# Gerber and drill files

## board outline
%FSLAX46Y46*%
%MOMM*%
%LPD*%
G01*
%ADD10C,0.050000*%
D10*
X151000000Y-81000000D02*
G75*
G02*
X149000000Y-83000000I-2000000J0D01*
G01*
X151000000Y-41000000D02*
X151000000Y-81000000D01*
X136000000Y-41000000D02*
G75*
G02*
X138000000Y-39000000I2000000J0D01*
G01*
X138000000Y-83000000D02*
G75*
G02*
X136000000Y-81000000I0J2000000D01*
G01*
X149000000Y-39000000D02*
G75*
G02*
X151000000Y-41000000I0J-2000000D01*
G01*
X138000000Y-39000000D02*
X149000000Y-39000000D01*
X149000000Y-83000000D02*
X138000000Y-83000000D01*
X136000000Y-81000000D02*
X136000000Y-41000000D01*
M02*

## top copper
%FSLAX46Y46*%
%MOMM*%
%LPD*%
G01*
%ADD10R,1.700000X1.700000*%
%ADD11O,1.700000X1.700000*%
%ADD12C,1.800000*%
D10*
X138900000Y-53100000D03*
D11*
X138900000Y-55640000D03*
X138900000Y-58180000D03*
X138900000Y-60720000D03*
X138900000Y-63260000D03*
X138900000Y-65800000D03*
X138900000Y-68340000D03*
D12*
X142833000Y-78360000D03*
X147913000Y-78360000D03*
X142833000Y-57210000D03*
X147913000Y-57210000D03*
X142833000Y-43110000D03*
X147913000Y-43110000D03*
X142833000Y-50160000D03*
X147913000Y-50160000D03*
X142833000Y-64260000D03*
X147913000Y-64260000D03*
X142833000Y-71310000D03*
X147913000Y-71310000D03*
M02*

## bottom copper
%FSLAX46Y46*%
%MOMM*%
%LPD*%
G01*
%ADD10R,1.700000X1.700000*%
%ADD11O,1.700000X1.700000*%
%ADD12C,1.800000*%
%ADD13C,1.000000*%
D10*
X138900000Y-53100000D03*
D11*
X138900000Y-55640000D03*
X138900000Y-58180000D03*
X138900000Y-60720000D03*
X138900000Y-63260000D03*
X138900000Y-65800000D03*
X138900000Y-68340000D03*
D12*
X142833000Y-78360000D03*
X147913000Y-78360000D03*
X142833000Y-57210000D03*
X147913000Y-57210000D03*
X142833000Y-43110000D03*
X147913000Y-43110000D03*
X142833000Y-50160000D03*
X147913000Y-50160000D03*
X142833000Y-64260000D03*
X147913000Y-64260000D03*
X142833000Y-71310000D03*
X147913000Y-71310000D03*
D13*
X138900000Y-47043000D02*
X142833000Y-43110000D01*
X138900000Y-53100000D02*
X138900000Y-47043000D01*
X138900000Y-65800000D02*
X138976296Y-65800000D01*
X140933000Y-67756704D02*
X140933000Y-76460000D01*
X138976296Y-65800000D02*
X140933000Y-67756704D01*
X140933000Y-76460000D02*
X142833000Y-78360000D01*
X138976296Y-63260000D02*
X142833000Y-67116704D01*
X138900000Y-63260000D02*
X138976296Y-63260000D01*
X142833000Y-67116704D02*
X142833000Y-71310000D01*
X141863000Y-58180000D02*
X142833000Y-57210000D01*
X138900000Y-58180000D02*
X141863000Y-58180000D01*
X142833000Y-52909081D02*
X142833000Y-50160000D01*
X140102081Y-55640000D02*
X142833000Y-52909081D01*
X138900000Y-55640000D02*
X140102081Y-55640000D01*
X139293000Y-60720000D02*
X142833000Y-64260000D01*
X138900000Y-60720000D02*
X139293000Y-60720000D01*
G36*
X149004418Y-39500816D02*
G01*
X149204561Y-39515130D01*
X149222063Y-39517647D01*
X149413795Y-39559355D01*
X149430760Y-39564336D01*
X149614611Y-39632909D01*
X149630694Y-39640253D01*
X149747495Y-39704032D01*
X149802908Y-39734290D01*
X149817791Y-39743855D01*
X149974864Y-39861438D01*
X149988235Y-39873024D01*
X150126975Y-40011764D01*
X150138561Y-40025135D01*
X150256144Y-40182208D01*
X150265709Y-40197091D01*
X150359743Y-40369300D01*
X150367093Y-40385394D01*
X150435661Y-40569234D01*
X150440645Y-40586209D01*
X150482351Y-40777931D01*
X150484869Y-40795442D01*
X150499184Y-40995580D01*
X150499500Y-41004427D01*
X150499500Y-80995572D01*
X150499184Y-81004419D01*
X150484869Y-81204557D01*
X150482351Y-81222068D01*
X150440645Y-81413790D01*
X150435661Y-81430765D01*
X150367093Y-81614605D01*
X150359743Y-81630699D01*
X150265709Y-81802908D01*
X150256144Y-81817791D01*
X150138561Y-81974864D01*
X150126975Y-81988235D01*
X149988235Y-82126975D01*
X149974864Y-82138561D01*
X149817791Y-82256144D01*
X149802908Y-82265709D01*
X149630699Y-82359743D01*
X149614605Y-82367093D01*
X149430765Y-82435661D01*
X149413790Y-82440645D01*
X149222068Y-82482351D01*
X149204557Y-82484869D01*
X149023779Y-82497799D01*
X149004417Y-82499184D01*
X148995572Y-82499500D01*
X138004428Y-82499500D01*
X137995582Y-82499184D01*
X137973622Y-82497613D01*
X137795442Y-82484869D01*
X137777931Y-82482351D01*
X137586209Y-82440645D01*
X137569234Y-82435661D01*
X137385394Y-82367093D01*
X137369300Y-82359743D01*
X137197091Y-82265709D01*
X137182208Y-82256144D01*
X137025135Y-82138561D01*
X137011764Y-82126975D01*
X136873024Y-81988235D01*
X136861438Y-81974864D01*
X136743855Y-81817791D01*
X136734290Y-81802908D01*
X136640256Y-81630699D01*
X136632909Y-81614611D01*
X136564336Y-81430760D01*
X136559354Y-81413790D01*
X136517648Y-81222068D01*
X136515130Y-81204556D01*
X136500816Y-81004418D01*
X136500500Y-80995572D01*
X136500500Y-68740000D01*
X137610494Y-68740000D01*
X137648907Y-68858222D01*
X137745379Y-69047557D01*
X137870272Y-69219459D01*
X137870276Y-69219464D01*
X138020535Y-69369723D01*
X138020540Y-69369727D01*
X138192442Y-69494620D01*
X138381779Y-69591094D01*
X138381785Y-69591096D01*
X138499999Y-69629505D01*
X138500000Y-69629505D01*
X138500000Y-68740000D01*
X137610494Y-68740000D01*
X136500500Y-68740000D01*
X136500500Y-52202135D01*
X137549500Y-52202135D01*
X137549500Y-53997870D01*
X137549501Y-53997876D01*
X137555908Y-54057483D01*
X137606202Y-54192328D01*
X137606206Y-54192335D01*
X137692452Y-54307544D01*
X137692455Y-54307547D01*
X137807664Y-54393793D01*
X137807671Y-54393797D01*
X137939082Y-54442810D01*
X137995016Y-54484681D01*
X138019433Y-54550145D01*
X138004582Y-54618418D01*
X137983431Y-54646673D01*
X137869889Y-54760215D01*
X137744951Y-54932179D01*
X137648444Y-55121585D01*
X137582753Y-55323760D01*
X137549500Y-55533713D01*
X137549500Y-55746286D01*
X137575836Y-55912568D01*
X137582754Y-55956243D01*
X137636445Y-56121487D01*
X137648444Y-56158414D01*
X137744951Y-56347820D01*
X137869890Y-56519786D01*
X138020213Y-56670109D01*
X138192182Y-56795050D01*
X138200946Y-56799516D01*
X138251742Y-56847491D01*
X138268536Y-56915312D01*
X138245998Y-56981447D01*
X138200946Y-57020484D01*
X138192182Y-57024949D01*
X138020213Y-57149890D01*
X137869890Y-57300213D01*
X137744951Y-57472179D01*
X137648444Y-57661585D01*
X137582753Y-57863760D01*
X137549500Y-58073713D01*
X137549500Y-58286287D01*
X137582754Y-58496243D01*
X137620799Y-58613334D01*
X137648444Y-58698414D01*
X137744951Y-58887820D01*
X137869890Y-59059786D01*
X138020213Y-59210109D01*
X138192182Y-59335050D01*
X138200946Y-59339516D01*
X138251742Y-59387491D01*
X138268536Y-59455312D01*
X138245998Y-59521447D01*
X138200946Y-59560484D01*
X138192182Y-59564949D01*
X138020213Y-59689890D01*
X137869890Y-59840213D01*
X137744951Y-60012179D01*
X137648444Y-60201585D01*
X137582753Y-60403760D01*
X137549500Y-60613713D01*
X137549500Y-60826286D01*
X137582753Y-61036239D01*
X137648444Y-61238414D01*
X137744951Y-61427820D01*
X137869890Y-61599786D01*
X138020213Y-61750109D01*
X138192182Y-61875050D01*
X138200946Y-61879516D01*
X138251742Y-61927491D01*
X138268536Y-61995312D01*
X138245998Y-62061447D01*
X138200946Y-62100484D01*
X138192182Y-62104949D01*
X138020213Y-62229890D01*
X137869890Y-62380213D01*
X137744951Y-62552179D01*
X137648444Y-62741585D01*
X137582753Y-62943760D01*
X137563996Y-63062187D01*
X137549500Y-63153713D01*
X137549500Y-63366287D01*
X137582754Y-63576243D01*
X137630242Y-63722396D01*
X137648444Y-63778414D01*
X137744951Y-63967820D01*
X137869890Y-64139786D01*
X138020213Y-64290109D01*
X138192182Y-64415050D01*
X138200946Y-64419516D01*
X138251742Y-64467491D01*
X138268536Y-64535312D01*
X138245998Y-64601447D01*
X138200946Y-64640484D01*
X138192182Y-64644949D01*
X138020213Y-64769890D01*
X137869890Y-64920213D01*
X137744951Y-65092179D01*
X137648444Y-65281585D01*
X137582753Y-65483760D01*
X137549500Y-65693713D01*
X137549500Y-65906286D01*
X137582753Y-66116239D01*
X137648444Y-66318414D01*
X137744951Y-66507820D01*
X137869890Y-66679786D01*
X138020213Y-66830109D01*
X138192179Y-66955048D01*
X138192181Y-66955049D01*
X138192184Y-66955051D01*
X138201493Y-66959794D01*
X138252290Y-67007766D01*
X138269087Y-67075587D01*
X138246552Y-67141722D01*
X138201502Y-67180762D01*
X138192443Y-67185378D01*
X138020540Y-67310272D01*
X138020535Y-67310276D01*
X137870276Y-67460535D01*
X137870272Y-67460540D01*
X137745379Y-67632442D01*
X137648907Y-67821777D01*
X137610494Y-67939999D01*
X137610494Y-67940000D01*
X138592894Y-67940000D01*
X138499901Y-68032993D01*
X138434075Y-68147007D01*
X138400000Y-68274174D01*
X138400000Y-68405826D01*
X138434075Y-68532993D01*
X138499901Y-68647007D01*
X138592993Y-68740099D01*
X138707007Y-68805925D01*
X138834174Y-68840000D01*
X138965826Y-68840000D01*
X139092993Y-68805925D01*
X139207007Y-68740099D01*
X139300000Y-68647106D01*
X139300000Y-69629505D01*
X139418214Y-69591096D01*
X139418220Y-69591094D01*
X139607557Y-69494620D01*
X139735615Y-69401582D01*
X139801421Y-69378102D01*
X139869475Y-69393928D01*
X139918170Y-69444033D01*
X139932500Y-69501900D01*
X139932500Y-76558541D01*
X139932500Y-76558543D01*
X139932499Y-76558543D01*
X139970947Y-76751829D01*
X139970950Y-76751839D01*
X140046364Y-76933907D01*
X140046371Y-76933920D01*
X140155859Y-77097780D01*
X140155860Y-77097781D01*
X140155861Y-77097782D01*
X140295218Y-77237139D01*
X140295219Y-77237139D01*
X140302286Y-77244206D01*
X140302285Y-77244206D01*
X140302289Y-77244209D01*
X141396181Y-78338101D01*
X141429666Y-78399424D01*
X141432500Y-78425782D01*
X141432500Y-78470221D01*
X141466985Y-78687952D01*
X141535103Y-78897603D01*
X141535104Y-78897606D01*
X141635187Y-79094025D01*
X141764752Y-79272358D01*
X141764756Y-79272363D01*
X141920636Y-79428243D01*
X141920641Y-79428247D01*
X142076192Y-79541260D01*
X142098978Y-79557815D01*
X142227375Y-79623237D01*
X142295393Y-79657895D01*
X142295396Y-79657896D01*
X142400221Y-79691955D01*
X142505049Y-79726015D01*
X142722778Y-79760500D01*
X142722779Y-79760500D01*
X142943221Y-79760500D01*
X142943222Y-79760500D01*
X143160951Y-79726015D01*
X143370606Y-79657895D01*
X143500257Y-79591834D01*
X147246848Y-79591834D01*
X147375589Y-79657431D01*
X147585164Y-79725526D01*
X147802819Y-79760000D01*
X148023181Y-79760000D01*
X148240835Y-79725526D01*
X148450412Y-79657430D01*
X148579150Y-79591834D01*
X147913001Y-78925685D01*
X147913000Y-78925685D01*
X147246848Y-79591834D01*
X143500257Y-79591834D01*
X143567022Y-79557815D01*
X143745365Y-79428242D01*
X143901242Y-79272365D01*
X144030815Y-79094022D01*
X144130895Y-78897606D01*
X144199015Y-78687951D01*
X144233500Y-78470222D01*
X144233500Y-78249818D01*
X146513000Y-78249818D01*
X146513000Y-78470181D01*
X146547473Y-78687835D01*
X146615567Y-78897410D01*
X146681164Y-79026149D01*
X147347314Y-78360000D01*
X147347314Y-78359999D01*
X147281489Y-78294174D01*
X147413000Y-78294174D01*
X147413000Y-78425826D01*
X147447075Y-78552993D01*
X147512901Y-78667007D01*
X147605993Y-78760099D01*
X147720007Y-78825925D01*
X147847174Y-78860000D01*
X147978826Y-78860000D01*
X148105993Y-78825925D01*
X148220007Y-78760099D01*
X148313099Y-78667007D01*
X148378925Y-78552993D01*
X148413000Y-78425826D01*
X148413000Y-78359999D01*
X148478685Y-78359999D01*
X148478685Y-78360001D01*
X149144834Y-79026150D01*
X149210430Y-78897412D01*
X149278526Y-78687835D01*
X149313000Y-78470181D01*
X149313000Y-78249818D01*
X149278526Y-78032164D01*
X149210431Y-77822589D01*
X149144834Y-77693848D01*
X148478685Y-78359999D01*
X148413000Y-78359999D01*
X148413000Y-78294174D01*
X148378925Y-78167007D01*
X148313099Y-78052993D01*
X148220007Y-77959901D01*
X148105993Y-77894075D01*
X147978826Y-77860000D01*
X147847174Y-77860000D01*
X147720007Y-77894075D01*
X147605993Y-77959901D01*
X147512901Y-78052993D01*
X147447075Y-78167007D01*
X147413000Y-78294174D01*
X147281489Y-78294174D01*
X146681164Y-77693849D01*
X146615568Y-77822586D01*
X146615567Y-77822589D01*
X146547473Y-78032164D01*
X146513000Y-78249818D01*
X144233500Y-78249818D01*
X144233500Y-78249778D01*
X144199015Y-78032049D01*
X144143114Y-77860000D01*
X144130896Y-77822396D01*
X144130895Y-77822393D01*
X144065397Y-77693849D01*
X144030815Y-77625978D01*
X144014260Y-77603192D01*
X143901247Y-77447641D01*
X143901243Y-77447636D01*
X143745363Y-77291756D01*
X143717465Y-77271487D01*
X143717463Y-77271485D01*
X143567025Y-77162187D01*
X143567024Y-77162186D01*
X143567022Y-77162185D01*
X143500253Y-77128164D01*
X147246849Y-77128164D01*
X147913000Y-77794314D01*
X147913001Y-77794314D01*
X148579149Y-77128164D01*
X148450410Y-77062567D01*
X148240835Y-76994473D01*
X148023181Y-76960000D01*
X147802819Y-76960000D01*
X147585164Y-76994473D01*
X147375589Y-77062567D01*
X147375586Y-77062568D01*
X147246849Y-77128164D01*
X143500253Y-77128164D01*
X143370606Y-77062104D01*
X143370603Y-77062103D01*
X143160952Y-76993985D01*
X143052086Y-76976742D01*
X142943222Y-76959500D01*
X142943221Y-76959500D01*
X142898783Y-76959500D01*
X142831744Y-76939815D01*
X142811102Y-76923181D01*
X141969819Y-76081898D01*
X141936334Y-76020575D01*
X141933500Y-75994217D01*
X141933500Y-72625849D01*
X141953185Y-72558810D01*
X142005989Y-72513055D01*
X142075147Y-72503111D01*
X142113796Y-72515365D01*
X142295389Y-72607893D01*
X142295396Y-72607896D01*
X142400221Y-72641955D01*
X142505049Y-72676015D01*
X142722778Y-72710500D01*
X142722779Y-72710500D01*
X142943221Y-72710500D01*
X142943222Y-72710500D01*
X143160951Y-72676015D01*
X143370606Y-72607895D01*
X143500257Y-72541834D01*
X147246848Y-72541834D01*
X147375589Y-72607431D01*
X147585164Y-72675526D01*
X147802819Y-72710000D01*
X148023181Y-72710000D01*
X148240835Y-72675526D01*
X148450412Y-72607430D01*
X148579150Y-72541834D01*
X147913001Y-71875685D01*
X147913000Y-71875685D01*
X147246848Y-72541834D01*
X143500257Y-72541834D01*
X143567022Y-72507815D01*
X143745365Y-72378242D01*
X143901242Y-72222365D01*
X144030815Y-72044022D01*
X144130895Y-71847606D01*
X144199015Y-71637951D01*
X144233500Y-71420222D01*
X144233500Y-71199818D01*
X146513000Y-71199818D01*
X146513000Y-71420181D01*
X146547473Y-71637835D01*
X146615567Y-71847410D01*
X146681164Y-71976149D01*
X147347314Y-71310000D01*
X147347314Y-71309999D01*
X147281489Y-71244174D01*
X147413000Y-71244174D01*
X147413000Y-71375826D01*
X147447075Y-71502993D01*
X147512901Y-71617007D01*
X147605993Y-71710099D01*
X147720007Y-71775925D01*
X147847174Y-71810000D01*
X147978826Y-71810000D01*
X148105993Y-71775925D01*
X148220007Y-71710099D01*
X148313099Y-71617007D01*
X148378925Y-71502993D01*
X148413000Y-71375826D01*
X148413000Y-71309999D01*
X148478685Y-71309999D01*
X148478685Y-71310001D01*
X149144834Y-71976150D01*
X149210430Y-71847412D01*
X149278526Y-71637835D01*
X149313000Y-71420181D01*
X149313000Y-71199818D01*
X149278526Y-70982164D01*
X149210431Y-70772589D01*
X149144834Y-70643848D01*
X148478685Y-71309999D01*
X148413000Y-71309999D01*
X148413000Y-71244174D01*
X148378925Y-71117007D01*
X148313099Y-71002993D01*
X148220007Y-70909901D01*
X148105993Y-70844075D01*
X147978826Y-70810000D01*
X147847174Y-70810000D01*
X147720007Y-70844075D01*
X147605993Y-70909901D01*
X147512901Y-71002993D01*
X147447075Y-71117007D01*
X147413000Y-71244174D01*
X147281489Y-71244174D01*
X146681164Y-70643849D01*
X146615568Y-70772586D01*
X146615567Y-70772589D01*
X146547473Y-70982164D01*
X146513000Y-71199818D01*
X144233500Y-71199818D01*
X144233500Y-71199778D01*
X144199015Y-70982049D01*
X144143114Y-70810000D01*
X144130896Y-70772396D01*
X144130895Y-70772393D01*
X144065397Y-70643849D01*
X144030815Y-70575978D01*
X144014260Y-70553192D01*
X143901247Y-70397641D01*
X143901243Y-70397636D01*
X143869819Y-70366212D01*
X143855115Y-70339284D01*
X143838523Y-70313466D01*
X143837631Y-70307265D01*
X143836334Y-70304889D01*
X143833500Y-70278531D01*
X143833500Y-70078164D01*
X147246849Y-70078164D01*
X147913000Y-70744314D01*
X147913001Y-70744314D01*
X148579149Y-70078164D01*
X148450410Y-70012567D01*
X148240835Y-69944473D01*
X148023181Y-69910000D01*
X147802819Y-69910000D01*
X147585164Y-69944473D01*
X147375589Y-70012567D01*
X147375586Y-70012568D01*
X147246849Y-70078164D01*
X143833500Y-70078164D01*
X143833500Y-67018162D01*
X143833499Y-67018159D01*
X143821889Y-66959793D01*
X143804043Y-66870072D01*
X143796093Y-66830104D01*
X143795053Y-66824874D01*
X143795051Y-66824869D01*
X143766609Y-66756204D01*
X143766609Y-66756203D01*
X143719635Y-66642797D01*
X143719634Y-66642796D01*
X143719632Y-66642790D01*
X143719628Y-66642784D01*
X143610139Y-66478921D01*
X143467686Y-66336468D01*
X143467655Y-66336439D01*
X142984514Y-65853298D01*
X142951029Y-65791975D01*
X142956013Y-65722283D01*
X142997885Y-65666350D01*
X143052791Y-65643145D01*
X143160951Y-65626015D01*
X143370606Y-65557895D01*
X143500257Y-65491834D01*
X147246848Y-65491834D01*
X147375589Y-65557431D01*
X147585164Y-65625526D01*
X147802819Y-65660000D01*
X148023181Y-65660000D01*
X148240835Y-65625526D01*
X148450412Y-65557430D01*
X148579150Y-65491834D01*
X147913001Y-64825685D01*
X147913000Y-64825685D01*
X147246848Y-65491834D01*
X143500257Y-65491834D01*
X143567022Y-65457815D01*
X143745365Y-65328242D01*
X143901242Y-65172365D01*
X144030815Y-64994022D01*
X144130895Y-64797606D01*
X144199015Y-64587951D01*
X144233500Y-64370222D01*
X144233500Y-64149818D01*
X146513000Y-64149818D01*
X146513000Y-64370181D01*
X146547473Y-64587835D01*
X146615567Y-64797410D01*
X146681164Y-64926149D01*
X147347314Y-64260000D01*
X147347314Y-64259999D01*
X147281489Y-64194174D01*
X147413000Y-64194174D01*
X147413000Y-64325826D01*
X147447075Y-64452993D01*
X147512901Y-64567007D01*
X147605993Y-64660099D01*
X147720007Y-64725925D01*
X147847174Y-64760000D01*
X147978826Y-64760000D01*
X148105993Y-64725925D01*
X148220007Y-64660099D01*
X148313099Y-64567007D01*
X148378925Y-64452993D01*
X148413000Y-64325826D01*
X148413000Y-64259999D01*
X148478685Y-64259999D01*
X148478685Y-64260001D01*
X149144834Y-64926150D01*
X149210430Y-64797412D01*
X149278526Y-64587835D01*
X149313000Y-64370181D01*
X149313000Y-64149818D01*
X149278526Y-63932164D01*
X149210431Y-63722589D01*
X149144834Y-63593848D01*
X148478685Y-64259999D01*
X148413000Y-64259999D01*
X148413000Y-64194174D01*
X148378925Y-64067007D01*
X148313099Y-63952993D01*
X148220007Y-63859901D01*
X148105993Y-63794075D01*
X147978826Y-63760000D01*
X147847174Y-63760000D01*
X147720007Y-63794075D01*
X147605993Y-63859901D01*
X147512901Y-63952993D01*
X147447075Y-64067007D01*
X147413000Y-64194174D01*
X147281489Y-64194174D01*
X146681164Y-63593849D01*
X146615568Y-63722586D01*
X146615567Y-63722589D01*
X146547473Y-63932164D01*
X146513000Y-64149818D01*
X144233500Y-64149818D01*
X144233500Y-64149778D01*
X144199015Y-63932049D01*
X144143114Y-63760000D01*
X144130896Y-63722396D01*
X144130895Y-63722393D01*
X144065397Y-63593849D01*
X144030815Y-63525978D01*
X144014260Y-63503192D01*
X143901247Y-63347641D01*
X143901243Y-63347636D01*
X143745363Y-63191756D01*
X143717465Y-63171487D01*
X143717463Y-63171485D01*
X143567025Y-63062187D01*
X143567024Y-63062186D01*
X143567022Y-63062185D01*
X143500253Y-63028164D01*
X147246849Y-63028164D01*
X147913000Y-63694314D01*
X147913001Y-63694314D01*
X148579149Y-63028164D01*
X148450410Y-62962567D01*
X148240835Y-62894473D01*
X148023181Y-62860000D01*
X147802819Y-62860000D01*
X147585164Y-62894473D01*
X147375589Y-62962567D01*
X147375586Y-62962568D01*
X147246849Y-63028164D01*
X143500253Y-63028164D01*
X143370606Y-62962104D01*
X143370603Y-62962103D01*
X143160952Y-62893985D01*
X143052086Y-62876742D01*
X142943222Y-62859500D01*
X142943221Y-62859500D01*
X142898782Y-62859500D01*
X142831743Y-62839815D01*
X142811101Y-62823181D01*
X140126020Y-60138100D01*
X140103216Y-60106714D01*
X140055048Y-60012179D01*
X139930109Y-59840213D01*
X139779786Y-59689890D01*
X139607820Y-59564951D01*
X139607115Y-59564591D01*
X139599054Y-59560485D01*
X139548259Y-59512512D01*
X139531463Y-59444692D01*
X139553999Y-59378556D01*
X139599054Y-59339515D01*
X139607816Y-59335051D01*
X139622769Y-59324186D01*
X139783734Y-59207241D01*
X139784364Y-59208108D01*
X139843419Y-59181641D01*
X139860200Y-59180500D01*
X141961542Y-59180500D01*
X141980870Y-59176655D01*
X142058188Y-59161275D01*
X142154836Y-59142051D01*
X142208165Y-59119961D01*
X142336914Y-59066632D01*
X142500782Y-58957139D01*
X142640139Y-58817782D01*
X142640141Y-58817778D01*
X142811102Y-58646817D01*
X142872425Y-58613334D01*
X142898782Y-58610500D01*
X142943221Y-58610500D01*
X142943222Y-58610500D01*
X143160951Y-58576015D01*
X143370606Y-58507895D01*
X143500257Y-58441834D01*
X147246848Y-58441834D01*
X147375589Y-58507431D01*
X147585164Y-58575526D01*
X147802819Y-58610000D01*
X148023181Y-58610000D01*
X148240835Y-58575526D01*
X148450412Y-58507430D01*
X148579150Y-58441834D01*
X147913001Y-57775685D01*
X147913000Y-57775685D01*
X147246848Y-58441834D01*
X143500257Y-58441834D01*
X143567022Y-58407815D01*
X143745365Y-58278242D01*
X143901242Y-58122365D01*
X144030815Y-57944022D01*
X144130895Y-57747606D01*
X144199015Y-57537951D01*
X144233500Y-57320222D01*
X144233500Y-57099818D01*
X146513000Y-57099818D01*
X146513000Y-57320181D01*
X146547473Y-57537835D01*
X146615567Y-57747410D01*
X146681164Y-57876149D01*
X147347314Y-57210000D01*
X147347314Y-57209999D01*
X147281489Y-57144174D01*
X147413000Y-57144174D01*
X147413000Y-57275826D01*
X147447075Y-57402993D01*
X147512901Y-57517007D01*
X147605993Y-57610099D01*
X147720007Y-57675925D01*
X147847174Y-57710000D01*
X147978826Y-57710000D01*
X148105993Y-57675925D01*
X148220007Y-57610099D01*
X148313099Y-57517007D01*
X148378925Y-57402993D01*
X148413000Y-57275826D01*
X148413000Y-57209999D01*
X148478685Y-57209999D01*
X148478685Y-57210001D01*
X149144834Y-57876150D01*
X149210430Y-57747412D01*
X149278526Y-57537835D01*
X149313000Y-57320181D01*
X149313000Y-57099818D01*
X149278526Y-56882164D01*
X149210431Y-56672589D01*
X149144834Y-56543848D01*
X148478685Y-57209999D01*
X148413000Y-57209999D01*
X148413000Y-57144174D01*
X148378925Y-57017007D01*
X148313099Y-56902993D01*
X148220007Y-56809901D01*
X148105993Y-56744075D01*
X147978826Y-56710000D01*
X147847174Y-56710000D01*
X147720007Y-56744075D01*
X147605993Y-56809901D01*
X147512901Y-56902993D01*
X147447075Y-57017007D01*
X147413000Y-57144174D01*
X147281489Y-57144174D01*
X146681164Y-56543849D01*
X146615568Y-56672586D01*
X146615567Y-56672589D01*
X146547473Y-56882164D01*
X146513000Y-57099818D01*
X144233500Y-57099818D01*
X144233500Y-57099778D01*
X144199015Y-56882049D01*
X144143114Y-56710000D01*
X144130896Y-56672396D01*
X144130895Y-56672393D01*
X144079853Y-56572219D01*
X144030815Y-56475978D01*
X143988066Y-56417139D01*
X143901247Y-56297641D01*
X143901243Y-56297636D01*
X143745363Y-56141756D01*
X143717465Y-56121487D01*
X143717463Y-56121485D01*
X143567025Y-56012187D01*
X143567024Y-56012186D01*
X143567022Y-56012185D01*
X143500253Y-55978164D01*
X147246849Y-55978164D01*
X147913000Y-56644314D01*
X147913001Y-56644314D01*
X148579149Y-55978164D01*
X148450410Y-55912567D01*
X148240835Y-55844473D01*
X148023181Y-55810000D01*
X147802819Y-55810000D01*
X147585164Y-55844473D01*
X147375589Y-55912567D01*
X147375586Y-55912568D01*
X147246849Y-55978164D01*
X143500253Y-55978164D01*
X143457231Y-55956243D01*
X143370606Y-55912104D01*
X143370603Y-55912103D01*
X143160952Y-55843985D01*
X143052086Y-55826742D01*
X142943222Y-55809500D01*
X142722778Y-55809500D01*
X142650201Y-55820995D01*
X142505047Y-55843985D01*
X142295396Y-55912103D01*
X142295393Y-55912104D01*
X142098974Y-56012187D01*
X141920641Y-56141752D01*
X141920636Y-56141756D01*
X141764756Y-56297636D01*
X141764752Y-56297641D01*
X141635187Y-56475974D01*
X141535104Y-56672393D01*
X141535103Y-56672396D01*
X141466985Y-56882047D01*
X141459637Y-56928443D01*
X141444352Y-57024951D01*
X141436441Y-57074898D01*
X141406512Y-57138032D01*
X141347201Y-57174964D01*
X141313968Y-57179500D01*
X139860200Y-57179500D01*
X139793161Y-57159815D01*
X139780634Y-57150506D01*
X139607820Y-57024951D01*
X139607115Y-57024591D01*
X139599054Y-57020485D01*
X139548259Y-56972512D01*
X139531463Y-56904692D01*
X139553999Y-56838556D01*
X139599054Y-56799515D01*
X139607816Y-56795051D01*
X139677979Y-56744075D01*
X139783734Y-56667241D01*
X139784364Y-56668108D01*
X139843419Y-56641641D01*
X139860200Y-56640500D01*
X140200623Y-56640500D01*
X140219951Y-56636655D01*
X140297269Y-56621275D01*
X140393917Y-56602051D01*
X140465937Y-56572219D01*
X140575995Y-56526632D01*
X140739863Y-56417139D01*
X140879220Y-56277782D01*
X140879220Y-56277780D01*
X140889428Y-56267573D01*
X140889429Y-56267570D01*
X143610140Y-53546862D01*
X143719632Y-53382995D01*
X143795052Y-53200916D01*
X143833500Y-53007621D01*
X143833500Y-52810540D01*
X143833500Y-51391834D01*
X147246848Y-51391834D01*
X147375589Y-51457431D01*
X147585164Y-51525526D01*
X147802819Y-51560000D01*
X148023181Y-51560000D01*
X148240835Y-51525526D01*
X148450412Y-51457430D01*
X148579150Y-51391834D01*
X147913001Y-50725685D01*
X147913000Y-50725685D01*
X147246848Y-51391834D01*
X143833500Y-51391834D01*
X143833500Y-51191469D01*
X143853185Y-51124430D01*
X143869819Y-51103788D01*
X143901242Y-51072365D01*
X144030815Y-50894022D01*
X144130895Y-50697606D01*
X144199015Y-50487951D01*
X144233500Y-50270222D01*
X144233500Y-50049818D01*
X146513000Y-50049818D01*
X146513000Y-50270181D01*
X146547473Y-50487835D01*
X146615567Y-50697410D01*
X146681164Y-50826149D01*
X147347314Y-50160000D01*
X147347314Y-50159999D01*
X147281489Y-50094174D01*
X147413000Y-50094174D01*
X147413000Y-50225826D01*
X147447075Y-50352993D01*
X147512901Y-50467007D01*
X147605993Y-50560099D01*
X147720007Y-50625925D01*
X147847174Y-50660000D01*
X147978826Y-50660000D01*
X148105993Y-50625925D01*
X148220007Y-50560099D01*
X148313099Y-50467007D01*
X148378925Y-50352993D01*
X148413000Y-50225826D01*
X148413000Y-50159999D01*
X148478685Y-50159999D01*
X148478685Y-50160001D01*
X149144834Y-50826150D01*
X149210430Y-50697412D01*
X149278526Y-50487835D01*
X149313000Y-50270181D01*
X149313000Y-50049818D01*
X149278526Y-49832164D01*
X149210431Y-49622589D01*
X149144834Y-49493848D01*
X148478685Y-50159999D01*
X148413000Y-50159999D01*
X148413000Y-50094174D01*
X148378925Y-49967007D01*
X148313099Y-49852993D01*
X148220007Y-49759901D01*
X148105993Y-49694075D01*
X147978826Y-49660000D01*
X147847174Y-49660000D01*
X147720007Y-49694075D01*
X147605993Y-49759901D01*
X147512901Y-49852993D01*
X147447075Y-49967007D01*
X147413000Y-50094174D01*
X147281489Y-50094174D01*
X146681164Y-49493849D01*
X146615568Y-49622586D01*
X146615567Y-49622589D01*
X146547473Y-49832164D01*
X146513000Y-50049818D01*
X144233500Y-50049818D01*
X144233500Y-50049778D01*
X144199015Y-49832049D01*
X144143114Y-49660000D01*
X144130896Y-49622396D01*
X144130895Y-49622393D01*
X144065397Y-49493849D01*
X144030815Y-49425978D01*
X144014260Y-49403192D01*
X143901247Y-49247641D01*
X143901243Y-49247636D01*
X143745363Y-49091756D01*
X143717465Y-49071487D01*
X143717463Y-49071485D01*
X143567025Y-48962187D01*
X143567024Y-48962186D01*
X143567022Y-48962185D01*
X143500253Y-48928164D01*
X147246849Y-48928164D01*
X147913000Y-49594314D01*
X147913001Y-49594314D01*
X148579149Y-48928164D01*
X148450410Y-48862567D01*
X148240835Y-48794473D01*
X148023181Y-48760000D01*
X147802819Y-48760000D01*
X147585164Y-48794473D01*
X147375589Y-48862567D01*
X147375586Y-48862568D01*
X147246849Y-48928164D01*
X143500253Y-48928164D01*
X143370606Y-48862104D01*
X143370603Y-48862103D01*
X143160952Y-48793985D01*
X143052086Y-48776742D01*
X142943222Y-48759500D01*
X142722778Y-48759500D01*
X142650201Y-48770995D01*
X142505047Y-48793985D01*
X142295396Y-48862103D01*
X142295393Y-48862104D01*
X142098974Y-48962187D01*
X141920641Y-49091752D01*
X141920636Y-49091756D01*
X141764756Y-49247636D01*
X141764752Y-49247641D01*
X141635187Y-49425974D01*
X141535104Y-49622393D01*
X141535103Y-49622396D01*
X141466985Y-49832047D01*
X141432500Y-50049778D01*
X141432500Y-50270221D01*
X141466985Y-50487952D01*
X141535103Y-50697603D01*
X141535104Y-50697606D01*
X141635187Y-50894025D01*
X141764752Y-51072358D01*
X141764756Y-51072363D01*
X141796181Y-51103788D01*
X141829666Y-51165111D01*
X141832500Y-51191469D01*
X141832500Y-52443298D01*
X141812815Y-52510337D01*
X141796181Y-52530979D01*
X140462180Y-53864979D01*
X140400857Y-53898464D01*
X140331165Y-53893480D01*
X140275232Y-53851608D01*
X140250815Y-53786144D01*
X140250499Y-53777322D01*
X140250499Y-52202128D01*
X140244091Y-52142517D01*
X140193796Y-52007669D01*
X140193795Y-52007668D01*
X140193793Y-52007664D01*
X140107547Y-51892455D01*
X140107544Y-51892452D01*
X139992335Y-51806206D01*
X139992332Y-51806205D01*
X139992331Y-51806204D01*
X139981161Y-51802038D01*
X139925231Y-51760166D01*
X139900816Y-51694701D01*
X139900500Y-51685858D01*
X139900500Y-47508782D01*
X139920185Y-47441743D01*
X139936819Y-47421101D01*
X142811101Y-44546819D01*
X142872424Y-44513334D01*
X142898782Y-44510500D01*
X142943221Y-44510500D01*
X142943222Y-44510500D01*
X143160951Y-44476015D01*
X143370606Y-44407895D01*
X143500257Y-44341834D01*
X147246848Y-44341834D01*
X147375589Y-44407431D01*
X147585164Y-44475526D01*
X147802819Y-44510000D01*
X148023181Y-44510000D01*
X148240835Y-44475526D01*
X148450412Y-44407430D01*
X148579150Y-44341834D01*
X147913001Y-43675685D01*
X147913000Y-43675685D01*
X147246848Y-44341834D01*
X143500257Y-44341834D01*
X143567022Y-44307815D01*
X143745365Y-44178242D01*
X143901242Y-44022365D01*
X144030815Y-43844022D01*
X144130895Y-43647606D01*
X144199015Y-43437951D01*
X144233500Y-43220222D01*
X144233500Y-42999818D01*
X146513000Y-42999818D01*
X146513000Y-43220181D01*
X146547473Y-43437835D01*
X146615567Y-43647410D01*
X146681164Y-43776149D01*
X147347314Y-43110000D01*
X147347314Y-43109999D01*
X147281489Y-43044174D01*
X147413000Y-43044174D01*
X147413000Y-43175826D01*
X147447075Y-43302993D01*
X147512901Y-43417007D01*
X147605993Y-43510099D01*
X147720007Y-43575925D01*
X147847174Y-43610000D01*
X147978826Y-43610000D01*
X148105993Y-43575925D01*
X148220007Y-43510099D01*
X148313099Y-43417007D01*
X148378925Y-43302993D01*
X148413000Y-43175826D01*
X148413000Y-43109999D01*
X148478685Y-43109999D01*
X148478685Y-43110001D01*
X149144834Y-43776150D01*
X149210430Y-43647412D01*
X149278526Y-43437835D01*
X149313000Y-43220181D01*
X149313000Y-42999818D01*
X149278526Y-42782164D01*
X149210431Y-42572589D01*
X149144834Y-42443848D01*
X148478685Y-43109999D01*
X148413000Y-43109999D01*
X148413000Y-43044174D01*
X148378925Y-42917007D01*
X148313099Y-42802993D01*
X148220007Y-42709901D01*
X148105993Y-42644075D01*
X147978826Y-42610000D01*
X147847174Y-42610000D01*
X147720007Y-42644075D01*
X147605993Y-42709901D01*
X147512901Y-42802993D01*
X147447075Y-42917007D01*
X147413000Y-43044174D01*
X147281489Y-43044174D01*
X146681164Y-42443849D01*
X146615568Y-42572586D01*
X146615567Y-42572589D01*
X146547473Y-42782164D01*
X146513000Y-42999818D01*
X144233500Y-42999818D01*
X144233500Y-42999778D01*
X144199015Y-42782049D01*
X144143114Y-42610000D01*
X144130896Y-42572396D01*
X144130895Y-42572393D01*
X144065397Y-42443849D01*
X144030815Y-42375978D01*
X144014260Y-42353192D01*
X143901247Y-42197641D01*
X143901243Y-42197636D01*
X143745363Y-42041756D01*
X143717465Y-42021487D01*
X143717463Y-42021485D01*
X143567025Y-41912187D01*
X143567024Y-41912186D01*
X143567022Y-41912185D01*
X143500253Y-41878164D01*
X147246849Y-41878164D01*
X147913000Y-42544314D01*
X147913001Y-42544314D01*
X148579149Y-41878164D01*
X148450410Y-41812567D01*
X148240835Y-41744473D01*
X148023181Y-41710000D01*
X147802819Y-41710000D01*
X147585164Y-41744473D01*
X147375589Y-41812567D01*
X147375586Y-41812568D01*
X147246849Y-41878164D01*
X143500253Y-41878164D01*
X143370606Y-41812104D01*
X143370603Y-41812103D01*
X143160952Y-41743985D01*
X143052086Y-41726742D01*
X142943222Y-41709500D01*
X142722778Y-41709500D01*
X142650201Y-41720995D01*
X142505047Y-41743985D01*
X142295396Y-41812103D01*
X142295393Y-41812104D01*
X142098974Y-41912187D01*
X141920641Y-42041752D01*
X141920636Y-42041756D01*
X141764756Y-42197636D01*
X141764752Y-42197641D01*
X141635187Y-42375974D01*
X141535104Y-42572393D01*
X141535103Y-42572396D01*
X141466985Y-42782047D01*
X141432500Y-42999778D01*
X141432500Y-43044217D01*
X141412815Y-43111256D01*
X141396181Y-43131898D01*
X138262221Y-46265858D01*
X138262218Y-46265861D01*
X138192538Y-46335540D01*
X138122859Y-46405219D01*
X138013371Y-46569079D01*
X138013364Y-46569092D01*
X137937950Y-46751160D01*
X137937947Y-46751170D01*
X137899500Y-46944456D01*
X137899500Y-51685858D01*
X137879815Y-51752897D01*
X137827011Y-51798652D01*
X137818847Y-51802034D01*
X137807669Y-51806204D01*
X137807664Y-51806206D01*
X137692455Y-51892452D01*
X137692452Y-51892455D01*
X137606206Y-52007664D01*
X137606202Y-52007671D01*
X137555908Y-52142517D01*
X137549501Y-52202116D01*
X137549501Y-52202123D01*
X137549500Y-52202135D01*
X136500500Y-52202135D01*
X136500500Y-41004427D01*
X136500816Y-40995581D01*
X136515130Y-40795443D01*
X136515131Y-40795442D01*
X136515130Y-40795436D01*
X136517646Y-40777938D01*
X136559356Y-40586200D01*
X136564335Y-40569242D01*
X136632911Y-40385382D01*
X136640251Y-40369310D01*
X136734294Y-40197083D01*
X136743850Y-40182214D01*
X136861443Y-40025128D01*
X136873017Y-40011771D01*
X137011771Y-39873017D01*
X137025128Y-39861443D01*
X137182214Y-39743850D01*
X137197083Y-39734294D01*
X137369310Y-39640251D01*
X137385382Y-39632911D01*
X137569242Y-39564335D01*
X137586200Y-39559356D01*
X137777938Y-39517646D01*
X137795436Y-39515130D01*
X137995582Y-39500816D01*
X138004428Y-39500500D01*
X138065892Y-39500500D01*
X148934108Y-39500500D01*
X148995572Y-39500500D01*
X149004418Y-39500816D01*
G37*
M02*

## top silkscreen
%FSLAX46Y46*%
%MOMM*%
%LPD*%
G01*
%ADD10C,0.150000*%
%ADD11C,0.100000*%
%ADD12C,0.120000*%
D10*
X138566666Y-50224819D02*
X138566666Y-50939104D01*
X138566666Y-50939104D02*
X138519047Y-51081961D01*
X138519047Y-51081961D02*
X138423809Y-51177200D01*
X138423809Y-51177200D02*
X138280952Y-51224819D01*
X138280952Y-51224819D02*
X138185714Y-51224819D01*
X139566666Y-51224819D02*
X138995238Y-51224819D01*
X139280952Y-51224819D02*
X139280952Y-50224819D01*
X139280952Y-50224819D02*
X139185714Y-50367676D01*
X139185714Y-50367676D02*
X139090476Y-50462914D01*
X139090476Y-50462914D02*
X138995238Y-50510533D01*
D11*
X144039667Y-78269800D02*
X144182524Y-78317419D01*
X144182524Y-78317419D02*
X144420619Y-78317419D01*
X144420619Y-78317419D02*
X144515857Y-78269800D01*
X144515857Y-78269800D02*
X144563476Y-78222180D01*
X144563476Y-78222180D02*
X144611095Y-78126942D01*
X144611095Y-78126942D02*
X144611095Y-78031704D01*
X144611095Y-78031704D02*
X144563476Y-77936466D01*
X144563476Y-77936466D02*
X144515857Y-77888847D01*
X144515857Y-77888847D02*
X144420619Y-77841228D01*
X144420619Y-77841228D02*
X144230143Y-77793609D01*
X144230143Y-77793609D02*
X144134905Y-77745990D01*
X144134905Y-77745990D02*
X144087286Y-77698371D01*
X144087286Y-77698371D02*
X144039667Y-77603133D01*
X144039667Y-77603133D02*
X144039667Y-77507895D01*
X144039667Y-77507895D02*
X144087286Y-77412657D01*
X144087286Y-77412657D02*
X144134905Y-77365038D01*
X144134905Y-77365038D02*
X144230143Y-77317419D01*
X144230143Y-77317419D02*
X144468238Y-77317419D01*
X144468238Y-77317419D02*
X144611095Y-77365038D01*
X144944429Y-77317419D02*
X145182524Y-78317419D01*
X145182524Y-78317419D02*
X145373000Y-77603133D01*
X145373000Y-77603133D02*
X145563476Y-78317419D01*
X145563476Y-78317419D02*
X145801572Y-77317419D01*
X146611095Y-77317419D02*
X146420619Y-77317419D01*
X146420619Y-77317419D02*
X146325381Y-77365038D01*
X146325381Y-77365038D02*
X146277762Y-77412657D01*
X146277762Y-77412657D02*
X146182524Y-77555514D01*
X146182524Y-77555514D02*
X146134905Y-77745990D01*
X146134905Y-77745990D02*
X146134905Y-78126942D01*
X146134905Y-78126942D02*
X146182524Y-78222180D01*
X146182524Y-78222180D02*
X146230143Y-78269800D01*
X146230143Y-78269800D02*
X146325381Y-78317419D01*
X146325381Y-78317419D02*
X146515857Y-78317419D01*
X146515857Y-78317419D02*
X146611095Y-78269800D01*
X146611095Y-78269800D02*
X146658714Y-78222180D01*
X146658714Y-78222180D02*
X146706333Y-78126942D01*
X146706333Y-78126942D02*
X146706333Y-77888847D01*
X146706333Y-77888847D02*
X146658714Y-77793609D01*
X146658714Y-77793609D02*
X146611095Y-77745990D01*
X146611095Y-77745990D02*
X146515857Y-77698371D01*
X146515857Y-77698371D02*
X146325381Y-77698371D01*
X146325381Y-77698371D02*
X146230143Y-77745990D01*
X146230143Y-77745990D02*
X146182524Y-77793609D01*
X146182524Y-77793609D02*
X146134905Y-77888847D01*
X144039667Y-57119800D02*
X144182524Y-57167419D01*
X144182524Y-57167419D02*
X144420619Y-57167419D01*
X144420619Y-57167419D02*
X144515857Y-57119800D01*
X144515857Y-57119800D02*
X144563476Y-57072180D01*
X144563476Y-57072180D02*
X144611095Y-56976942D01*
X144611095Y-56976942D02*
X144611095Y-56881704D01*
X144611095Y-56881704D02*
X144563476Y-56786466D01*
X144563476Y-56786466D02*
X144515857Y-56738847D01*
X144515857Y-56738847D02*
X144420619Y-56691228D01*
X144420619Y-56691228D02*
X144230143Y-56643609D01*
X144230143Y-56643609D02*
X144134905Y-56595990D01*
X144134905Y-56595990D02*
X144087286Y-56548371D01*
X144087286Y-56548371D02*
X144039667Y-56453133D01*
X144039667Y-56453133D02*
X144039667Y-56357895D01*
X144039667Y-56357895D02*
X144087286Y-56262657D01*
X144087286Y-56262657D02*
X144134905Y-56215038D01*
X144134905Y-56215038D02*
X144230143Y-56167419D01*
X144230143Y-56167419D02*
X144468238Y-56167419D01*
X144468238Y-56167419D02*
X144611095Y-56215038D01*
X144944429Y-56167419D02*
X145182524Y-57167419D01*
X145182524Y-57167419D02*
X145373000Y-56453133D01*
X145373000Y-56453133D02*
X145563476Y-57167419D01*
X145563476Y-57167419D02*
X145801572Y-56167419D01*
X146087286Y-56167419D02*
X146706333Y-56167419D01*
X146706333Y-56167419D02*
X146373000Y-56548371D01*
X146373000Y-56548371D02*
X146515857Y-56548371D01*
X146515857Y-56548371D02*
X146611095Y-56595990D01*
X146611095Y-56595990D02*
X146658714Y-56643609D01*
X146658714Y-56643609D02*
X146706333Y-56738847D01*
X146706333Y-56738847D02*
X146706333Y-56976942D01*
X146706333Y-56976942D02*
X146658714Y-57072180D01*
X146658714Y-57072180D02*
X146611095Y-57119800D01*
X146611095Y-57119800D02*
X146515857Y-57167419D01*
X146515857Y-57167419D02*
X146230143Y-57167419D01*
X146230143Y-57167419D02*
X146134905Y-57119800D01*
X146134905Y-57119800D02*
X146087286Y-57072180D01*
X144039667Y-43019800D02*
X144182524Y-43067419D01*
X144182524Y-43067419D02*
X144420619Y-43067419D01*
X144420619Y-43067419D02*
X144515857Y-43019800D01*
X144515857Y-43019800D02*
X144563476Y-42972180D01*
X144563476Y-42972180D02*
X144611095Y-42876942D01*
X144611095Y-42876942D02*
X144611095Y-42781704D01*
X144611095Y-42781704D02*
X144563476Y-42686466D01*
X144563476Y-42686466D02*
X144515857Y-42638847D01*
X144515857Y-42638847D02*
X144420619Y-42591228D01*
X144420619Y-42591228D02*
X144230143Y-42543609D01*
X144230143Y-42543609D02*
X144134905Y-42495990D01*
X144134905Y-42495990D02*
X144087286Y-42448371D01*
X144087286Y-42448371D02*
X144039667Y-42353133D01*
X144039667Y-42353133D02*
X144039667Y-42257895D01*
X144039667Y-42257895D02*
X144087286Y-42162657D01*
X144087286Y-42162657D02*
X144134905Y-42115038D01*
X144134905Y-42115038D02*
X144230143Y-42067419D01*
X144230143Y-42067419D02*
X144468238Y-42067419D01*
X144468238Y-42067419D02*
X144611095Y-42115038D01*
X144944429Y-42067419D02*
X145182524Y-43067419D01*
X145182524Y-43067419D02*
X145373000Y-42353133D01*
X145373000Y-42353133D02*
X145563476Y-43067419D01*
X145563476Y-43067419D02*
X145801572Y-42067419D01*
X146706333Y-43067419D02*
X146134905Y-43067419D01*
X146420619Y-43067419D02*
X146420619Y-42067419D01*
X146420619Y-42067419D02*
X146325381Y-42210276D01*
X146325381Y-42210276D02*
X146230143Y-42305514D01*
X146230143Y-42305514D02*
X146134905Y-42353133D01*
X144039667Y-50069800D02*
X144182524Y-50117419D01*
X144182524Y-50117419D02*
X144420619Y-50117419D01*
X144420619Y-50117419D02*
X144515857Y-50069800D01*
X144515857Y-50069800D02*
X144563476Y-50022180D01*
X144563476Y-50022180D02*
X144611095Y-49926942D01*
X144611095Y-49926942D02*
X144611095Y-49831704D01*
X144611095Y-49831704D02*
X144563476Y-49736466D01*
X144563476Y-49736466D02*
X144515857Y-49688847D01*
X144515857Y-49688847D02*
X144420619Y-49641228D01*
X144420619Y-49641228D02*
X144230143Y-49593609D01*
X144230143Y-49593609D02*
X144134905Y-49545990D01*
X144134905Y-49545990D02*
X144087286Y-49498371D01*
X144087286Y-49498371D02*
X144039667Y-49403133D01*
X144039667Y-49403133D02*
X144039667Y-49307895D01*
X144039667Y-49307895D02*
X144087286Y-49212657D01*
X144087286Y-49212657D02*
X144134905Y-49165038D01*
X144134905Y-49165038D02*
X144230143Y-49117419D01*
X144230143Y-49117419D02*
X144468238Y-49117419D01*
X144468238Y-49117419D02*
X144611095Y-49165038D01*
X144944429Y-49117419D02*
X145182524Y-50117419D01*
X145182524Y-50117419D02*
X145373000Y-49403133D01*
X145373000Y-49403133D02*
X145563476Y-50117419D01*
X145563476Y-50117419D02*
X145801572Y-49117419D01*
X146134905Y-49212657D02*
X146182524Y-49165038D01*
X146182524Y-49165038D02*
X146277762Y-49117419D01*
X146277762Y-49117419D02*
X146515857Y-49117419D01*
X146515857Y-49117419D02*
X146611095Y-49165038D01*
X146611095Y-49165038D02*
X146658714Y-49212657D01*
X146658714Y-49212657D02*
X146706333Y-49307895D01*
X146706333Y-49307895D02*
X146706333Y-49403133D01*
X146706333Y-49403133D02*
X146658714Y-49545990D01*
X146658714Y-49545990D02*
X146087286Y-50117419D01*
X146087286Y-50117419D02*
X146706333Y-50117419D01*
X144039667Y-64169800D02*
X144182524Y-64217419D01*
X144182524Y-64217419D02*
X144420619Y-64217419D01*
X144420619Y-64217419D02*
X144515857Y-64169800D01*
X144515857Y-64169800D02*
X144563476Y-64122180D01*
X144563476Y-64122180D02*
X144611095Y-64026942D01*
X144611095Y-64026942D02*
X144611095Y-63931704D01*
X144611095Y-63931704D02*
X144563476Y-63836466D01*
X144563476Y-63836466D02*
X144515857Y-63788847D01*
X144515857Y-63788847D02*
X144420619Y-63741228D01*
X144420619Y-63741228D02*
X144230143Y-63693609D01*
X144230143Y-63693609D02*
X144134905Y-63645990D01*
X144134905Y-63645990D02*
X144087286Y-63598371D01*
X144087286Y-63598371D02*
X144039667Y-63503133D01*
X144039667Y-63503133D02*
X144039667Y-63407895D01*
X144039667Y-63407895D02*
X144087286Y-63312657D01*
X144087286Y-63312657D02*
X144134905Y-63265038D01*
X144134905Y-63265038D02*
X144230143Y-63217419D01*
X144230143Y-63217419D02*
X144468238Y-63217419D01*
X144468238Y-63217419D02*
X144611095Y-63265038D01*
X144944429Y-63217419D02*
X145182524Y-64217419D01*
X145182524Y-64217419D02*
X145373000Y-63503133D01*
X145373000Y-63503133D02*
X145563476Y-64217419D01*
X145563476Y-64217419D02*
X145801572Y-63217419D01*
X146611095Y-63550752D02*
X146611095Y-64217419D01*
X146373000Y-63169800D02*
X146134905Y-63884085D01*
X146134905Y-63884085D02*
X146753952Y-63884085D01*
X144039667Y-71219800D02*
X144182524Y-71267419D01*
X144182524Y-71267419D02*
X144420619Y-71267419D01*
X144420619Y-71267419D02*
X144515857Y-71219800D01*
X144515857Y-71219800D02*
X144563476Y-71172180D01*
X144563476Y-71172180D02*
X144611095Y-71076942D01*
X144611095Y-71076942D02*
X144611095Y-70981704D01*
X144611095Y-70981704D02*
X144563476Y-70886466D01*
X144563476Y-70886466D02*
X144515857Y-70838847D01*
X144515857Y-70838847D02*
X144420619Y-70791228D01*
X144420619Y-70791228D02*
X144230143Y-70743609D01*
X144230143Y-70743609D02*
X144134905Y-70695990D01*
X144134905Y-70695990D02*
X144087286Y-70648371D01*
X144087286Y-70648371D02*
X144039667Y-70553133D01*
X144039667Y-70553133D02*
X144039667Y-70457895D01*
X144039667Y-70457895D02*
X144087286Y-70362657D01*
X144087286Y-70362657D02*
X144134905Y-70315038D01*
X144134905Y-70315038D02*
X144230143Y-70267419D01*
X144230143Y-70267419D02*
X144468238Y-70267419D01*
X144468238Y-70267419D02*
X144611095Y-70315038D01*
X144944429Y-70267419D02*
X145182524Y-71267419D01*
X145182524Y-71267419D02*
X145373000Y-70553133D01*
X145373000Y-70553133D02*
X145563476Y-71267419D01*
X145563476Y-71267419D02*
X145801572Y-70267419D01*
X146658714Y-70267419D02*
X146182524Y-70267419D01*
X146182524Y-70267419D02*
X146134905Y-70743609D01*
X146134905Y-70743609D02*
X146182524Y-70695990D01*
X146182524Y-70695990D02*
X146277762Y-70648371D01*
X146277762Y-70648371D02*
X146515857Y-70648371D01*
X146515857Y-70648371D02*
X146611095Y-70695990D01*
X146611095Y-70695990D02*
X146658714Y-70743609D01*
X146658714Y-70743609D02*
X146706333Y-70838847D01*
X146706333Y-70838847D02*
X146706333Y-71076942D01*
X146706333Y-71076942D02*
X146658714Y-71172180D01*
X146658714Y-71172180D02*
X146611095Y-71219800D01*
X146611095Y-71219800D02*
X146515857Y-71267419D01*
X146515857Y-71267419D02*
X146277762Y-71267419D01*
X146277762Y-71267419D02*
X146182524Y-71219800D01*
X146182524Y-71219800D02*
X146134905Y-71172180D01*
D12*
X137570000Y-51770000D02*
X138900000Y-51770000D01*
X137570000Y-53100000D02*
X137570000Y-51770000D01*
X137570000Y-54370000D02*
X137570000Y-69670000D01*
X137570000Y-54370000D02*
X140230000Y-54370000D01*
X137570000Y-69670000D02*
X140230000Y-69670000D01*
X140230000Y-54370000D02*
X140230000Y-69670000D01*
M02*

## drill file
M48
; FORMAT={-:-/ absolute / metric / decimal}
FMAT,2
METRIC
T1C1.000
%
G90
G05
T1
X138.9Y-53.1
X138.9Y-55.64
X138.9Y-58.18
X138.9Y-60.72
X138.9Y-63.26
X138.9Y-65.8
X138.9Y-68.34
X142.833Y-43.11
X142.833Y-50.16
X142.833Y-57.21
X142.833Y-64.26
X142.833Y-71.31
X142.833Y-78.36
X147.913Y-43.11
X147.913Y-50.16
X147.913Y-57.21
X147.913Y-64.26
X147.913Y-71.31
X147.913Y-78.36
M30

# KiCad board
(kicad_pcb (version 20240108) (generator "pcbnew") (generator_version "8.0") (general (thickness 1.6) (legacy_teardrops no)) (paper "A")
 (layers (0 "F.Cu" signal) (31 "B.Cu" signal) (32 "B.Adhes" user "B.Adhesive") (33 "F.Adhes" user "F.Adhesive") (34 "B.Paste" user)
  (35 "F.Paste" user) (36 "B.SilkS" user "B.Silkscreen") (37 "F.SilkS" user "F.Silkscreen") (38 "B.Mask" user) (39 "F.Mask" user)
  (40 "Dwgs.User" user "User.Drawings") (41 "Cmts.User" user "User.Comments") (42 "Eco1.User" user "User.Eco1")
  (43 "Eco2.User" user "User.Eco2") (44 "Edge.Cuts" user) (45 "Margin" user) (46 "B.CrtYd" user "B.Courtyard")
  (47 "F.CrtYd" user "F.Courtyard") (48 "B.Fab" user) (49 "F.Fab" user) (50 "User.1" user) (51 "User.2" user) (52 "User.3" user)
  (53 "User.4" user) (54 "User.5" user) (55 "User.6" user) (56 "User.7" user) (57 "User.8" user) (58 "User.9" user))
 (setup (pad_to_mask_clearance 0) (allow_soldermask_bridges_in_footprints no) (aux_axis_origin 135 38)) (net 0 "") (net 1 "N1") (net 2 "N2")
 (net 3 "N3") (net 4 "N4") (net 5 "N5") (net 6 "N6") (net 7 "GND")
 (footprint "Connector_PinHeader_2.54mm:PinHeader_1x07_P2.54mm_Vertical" (layer "F.Cu") (at 138.9 53.1)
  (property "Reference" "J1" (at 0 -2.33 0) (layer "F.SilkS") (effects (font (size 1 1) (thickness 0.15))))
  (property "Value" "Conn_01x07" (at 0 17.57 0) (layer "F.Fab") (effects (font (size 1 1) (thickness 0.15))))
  (fp_line (start -1.33 -1.33) (end 0 -1.33) (stroke (width 0.12) (type solid)) (layer "F.SilkS"))
  (fp_line (start -1.33 0) (end -1.33 -1.33) (stroke (width 0.12) (type solid)) (layer "F.SilkS"))
  (fp_line (start -1.33 1.27) (end -1.33 16.57) (stroke (width 0.12) (type solid)) (layer "F.SilkS"))
  (fp_line (start -1.33 1.27) (end 1.33 1.27) (stroke (width 0.12) (type solid)) (layer "F.SilkS"))
  (fp_line (start -1.33 16.57) (end 1.33 16.57) (stroke (width 0.12) (type solid)) (layer "F.SilkS"))
  (fp_line (start 1.33 1.27) (end 1.33 16.57) (stroke (width 0.12) (type solid)) (layer "F.SilkS"))
  (pad "1" thru_hole rect (at 0 0) (size 1.7 1.7) (drill 1) (layers "*.Cu" "*.Mask") (remove_unused_layers no) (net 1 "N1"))
  (pad "2" thru_hole oval (at 0 2.54) (size 1.7 1.7) (drill 1) (layers "*.Cu" "*.Mask") (remove_unused_layers no) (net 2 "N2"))
  (pad "3" thru_hole oval (at 0 5.08) (size 1.7 1.7) (drill 1) (layers "*.Cu" "*.Mask") (remove_unused_layers no) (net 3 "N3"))
  (pad "4" thru_hole oval (at 0 7.62) (size 1.7 1.7) (drill 1) (layers "*.Cu" "*.Mask") (remove_unused_layers no) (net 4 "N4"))
  (pad "5" thru_hole oval (at 0 10.16) (size 1.7 1.7) (drill 1) (layers "*.Cu" "*.Mask") (remove_unused_layers no) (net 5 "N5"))
  (pad "6" thru_hole oval (at 0 12.7) (size 1.7 1.7) (drill 1) (layers "*.Cu" "*.Mask") (remove_unused_layers no) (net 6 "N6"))
  (pad "7" thru_hole oval (at 0 15.24) (size 1.7 1.7) (drill 1) (layers "*.Cu" "*.Mask") (remove_unused_layers no) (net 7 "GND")))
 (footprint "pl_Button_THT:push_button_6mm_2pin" (layer "F.Cu") (at 145.373 78.36)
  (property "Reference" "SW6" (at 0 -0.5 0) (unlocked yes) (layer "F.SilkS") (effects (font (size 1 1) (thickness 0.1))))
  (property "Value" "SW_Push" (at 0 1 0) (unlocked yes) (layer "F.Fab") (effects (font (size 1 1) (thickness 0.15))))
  (pad "1" thru_hole circle (at -2.54 0) (size 1.8 1.8) (drill 1) (layers "*.Cu" "*.Mask") (remove_unused_layers no) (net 6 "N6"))
  (pad "2" thru_hole circle (at 2.54 0) (size 1.8 1.8) (drill 1) (layers "*.Cu" "*.Mask") (remove_unused_layers no) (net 7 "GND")))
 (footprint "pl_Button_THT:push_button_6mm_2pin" (layer "F.Cu") (at 145.373 57.21)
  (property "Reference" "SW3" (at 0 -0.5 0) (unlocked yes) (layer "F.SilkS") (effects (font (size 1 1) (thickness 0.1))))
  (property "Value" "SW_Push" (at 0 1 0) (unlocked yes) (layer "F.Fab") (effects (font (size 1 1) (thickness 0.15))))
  (pad "1" thru_hole circle (at -2.54 0) (size 1.8 1.8) (drill 1) (layers "*.Cu" "*.Mask") (remove_unused_layers no) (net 3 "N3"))
  (pad "2" thru_hole circle (at 2.54 0) (size 1.8 1.8) (drill 1) (layers "*.Cu" "*.Mask") (remove_unused_layers no) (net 7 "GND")))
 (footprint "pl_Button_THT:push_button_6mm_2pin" (layer "F.Cu") (at 145.373 43.11)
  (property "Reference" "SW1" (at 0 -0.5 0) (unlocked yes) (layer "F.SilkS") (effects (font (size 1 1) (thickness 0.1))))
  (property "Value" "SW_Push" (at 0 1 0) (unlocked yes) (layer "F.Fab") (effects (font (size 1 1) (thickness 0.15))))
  (pad "1" thru_hole circle (at -2.54 0) (size 1.8 1.8) (drill 1) (layers "*.Cu" "*.Mask") (remove_unused_layers no) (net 1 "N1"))
  (pad "2" thru_hole circle (at 2.54 0) (size 1.8 1.8) (drill 1) (layers "*.Cu" "*.Mask") (remove_unused_layers no) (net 7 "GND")))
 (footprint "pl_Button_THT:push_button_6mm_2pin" (layer "F.Cu") (at 145.373 50.16)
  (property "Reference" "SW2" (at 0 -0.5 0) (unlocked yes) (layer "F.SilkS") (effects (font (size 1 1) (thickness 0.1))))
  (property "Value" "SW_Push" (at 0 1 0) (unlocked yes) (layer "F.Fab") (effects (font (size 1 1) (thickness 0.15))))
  (pad "1" thru_hole circle (at -2.54 0) (size 1.8 1.8) (drill 1) (layers "*.Cu" "*.Mask") (remove_unused_layers no) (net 2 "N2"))
  (pad "2" thru_hole circle (at 2.54 0) (size 1.8 1.8) (drill 1) (layers "*.Cu" "*.Mask") (remove_unused_layers no) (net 7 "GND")))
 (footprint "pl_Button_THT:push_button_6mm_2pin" (layer "F.Cu") (at 145.373 64.26)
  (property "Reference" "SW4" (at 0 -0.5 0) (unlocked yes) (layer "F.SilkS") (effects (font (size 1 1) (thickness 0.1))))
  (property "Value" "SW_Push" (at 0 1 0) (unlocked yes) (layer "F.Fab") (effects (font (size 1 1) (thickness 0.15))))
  (pad "1" thru_hole circle (at -2.54 0) (size 1.8 1.8) (drill 1) (layers "*.Cu" "*.Mask") (remove_unused_layers no) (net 4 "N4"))
  (pad "2" thru_hole circle (at 2.54 0) (size 1.8 1.8) (drill 1) (layers "*.Cu" "*.Mask") (remove_unused_layers no) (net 7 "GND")))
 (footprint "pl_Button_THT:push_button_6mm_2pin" (layer "F.Cu") (at 145.373 71.31)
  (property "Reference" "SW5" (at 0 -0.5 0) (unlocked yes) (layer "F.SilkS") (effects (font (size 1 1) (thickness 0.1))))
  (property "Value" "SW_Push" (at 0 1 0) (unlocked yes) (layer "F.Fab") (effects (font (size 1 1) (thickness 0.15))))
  (pad "1" thru_hole circle (at -2.54 0) (size 1.8 1.8) (drill 1) (layers "*.Cu" "*.Mask") (remove_unused_layers no) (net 5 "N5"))
  (pad "2" thru_hole circle (at 2.54 0) (size 1.8 1.8) (drill 1) (layers "*.Cu" "*.Mask") (remove_unused_layers no) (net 7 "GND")))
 (gr_arc (start 151 81) (mid 150.414214 82.414214) (end 149 83) (stroke (width 0.05) (type default)) (layer "Edge.Cuts"))
 (gr_line (start 151 41) (end 151 81) (stroke (width 0.05) (type default)) (layer "Edge.Cuts"))
 (gr_arc (start 136 41) (mid 136.585786 39.585786) (end 138 39) (stroke (width 0.05) (type default)) (layer "Edge.Cuts"))
 (gr_arc (start 138 83) (mid 136.585786 82.414214) (end 136 81) (stroke (width 0.05) (type default)) (layer "Edge.Cuts"))
 (gr_arc (start 149 39) (mid 150.414214 39.585786) (end 151 41) (stroke (width 0.05) (type default)) (layer "Edge.Cuts"))
 (gr_line (start 138 39) (end 149 39) (stroke (width 0.05) (type default)) (layer "Edge.Cuts"))
 (gr_line (start 149 83) (end 138 83) (stroke (width 0.05) (type default)) (layer "Edge.Cuts"))
 (gr_line (start 136 81) (end 136 41) (stroke (width 0.05) (type default)) (layer "Edge.Cuts"))
 (segment (start 138.9 47.043) (end 142.833 43.11) (width 1) (layer "B.Cu") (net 1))
 (segment (start 138.9 53.1) (end 138.9 47.043) (width 1) (layer "B.Cu") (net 1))
 (segment (start 138.9 65.8) (end 138.976296 65.8) (width 1) (layer "B.Cu") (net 6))
 (segment (start 140.933 67.756704) (end 140.933 76.46) (width 1) (layer "B.Cu") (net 6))
 (segment (start 138.976296 65.8) (end 140.933 67.756704) (width 1) (layer "B.Cu") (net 6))
 (segment (start 140.933 76.46) (end 142.833 78.36) (width 1) (layer "B.Cu") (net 6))
 (segment (start 138.976296 63.26) (end 142.833 67.116704) (width 1) (layer "B.Cu") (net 5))
 (segment (start 138.9 63.26) (end 138.976296 63.26) (width 1) (layer "B.Cu") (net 5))
 (segment (start 142.833 67.116704) (end 142.833 71.31) (width 1) (layer "B.Cu") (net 5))
 (segment (start 141.863 58.18) (end 142.833 57.21) (width 1) (layer "B.Cu") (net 3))
 (segment (start 138.9 58.18) (end 141.863 58.18) (width 1) (layer "B.Cu") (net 3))
 (segment (start 142.833 52.909081) (end 142.833 50.16) (width 1) (layer "B.Cu") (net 2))
 (segment (start 140.102081 55.64) (end 142.833 52.909081) (width 1) (layer "B.Cu") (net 2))
 (segment (start 138.9 55.64) (end 140.102081 55.64) (width 1) (layer "B.Cu") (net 2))
 (segment (start 139.293 60.72) (end 142.833 64.26) (width 1) (layer "B.Cu") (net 4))
 (segment (start 138.9 60.72) (end 139.293 60.72) (width 1) (layer "B.Cu") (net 4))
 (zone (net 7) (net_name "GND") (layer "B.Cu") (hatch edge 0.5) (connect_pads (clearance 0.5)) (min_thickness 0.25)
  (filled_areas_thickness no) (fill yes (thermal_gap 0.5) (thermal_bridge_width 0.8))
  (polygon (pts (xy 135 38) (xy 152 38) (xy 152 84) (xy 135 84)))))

